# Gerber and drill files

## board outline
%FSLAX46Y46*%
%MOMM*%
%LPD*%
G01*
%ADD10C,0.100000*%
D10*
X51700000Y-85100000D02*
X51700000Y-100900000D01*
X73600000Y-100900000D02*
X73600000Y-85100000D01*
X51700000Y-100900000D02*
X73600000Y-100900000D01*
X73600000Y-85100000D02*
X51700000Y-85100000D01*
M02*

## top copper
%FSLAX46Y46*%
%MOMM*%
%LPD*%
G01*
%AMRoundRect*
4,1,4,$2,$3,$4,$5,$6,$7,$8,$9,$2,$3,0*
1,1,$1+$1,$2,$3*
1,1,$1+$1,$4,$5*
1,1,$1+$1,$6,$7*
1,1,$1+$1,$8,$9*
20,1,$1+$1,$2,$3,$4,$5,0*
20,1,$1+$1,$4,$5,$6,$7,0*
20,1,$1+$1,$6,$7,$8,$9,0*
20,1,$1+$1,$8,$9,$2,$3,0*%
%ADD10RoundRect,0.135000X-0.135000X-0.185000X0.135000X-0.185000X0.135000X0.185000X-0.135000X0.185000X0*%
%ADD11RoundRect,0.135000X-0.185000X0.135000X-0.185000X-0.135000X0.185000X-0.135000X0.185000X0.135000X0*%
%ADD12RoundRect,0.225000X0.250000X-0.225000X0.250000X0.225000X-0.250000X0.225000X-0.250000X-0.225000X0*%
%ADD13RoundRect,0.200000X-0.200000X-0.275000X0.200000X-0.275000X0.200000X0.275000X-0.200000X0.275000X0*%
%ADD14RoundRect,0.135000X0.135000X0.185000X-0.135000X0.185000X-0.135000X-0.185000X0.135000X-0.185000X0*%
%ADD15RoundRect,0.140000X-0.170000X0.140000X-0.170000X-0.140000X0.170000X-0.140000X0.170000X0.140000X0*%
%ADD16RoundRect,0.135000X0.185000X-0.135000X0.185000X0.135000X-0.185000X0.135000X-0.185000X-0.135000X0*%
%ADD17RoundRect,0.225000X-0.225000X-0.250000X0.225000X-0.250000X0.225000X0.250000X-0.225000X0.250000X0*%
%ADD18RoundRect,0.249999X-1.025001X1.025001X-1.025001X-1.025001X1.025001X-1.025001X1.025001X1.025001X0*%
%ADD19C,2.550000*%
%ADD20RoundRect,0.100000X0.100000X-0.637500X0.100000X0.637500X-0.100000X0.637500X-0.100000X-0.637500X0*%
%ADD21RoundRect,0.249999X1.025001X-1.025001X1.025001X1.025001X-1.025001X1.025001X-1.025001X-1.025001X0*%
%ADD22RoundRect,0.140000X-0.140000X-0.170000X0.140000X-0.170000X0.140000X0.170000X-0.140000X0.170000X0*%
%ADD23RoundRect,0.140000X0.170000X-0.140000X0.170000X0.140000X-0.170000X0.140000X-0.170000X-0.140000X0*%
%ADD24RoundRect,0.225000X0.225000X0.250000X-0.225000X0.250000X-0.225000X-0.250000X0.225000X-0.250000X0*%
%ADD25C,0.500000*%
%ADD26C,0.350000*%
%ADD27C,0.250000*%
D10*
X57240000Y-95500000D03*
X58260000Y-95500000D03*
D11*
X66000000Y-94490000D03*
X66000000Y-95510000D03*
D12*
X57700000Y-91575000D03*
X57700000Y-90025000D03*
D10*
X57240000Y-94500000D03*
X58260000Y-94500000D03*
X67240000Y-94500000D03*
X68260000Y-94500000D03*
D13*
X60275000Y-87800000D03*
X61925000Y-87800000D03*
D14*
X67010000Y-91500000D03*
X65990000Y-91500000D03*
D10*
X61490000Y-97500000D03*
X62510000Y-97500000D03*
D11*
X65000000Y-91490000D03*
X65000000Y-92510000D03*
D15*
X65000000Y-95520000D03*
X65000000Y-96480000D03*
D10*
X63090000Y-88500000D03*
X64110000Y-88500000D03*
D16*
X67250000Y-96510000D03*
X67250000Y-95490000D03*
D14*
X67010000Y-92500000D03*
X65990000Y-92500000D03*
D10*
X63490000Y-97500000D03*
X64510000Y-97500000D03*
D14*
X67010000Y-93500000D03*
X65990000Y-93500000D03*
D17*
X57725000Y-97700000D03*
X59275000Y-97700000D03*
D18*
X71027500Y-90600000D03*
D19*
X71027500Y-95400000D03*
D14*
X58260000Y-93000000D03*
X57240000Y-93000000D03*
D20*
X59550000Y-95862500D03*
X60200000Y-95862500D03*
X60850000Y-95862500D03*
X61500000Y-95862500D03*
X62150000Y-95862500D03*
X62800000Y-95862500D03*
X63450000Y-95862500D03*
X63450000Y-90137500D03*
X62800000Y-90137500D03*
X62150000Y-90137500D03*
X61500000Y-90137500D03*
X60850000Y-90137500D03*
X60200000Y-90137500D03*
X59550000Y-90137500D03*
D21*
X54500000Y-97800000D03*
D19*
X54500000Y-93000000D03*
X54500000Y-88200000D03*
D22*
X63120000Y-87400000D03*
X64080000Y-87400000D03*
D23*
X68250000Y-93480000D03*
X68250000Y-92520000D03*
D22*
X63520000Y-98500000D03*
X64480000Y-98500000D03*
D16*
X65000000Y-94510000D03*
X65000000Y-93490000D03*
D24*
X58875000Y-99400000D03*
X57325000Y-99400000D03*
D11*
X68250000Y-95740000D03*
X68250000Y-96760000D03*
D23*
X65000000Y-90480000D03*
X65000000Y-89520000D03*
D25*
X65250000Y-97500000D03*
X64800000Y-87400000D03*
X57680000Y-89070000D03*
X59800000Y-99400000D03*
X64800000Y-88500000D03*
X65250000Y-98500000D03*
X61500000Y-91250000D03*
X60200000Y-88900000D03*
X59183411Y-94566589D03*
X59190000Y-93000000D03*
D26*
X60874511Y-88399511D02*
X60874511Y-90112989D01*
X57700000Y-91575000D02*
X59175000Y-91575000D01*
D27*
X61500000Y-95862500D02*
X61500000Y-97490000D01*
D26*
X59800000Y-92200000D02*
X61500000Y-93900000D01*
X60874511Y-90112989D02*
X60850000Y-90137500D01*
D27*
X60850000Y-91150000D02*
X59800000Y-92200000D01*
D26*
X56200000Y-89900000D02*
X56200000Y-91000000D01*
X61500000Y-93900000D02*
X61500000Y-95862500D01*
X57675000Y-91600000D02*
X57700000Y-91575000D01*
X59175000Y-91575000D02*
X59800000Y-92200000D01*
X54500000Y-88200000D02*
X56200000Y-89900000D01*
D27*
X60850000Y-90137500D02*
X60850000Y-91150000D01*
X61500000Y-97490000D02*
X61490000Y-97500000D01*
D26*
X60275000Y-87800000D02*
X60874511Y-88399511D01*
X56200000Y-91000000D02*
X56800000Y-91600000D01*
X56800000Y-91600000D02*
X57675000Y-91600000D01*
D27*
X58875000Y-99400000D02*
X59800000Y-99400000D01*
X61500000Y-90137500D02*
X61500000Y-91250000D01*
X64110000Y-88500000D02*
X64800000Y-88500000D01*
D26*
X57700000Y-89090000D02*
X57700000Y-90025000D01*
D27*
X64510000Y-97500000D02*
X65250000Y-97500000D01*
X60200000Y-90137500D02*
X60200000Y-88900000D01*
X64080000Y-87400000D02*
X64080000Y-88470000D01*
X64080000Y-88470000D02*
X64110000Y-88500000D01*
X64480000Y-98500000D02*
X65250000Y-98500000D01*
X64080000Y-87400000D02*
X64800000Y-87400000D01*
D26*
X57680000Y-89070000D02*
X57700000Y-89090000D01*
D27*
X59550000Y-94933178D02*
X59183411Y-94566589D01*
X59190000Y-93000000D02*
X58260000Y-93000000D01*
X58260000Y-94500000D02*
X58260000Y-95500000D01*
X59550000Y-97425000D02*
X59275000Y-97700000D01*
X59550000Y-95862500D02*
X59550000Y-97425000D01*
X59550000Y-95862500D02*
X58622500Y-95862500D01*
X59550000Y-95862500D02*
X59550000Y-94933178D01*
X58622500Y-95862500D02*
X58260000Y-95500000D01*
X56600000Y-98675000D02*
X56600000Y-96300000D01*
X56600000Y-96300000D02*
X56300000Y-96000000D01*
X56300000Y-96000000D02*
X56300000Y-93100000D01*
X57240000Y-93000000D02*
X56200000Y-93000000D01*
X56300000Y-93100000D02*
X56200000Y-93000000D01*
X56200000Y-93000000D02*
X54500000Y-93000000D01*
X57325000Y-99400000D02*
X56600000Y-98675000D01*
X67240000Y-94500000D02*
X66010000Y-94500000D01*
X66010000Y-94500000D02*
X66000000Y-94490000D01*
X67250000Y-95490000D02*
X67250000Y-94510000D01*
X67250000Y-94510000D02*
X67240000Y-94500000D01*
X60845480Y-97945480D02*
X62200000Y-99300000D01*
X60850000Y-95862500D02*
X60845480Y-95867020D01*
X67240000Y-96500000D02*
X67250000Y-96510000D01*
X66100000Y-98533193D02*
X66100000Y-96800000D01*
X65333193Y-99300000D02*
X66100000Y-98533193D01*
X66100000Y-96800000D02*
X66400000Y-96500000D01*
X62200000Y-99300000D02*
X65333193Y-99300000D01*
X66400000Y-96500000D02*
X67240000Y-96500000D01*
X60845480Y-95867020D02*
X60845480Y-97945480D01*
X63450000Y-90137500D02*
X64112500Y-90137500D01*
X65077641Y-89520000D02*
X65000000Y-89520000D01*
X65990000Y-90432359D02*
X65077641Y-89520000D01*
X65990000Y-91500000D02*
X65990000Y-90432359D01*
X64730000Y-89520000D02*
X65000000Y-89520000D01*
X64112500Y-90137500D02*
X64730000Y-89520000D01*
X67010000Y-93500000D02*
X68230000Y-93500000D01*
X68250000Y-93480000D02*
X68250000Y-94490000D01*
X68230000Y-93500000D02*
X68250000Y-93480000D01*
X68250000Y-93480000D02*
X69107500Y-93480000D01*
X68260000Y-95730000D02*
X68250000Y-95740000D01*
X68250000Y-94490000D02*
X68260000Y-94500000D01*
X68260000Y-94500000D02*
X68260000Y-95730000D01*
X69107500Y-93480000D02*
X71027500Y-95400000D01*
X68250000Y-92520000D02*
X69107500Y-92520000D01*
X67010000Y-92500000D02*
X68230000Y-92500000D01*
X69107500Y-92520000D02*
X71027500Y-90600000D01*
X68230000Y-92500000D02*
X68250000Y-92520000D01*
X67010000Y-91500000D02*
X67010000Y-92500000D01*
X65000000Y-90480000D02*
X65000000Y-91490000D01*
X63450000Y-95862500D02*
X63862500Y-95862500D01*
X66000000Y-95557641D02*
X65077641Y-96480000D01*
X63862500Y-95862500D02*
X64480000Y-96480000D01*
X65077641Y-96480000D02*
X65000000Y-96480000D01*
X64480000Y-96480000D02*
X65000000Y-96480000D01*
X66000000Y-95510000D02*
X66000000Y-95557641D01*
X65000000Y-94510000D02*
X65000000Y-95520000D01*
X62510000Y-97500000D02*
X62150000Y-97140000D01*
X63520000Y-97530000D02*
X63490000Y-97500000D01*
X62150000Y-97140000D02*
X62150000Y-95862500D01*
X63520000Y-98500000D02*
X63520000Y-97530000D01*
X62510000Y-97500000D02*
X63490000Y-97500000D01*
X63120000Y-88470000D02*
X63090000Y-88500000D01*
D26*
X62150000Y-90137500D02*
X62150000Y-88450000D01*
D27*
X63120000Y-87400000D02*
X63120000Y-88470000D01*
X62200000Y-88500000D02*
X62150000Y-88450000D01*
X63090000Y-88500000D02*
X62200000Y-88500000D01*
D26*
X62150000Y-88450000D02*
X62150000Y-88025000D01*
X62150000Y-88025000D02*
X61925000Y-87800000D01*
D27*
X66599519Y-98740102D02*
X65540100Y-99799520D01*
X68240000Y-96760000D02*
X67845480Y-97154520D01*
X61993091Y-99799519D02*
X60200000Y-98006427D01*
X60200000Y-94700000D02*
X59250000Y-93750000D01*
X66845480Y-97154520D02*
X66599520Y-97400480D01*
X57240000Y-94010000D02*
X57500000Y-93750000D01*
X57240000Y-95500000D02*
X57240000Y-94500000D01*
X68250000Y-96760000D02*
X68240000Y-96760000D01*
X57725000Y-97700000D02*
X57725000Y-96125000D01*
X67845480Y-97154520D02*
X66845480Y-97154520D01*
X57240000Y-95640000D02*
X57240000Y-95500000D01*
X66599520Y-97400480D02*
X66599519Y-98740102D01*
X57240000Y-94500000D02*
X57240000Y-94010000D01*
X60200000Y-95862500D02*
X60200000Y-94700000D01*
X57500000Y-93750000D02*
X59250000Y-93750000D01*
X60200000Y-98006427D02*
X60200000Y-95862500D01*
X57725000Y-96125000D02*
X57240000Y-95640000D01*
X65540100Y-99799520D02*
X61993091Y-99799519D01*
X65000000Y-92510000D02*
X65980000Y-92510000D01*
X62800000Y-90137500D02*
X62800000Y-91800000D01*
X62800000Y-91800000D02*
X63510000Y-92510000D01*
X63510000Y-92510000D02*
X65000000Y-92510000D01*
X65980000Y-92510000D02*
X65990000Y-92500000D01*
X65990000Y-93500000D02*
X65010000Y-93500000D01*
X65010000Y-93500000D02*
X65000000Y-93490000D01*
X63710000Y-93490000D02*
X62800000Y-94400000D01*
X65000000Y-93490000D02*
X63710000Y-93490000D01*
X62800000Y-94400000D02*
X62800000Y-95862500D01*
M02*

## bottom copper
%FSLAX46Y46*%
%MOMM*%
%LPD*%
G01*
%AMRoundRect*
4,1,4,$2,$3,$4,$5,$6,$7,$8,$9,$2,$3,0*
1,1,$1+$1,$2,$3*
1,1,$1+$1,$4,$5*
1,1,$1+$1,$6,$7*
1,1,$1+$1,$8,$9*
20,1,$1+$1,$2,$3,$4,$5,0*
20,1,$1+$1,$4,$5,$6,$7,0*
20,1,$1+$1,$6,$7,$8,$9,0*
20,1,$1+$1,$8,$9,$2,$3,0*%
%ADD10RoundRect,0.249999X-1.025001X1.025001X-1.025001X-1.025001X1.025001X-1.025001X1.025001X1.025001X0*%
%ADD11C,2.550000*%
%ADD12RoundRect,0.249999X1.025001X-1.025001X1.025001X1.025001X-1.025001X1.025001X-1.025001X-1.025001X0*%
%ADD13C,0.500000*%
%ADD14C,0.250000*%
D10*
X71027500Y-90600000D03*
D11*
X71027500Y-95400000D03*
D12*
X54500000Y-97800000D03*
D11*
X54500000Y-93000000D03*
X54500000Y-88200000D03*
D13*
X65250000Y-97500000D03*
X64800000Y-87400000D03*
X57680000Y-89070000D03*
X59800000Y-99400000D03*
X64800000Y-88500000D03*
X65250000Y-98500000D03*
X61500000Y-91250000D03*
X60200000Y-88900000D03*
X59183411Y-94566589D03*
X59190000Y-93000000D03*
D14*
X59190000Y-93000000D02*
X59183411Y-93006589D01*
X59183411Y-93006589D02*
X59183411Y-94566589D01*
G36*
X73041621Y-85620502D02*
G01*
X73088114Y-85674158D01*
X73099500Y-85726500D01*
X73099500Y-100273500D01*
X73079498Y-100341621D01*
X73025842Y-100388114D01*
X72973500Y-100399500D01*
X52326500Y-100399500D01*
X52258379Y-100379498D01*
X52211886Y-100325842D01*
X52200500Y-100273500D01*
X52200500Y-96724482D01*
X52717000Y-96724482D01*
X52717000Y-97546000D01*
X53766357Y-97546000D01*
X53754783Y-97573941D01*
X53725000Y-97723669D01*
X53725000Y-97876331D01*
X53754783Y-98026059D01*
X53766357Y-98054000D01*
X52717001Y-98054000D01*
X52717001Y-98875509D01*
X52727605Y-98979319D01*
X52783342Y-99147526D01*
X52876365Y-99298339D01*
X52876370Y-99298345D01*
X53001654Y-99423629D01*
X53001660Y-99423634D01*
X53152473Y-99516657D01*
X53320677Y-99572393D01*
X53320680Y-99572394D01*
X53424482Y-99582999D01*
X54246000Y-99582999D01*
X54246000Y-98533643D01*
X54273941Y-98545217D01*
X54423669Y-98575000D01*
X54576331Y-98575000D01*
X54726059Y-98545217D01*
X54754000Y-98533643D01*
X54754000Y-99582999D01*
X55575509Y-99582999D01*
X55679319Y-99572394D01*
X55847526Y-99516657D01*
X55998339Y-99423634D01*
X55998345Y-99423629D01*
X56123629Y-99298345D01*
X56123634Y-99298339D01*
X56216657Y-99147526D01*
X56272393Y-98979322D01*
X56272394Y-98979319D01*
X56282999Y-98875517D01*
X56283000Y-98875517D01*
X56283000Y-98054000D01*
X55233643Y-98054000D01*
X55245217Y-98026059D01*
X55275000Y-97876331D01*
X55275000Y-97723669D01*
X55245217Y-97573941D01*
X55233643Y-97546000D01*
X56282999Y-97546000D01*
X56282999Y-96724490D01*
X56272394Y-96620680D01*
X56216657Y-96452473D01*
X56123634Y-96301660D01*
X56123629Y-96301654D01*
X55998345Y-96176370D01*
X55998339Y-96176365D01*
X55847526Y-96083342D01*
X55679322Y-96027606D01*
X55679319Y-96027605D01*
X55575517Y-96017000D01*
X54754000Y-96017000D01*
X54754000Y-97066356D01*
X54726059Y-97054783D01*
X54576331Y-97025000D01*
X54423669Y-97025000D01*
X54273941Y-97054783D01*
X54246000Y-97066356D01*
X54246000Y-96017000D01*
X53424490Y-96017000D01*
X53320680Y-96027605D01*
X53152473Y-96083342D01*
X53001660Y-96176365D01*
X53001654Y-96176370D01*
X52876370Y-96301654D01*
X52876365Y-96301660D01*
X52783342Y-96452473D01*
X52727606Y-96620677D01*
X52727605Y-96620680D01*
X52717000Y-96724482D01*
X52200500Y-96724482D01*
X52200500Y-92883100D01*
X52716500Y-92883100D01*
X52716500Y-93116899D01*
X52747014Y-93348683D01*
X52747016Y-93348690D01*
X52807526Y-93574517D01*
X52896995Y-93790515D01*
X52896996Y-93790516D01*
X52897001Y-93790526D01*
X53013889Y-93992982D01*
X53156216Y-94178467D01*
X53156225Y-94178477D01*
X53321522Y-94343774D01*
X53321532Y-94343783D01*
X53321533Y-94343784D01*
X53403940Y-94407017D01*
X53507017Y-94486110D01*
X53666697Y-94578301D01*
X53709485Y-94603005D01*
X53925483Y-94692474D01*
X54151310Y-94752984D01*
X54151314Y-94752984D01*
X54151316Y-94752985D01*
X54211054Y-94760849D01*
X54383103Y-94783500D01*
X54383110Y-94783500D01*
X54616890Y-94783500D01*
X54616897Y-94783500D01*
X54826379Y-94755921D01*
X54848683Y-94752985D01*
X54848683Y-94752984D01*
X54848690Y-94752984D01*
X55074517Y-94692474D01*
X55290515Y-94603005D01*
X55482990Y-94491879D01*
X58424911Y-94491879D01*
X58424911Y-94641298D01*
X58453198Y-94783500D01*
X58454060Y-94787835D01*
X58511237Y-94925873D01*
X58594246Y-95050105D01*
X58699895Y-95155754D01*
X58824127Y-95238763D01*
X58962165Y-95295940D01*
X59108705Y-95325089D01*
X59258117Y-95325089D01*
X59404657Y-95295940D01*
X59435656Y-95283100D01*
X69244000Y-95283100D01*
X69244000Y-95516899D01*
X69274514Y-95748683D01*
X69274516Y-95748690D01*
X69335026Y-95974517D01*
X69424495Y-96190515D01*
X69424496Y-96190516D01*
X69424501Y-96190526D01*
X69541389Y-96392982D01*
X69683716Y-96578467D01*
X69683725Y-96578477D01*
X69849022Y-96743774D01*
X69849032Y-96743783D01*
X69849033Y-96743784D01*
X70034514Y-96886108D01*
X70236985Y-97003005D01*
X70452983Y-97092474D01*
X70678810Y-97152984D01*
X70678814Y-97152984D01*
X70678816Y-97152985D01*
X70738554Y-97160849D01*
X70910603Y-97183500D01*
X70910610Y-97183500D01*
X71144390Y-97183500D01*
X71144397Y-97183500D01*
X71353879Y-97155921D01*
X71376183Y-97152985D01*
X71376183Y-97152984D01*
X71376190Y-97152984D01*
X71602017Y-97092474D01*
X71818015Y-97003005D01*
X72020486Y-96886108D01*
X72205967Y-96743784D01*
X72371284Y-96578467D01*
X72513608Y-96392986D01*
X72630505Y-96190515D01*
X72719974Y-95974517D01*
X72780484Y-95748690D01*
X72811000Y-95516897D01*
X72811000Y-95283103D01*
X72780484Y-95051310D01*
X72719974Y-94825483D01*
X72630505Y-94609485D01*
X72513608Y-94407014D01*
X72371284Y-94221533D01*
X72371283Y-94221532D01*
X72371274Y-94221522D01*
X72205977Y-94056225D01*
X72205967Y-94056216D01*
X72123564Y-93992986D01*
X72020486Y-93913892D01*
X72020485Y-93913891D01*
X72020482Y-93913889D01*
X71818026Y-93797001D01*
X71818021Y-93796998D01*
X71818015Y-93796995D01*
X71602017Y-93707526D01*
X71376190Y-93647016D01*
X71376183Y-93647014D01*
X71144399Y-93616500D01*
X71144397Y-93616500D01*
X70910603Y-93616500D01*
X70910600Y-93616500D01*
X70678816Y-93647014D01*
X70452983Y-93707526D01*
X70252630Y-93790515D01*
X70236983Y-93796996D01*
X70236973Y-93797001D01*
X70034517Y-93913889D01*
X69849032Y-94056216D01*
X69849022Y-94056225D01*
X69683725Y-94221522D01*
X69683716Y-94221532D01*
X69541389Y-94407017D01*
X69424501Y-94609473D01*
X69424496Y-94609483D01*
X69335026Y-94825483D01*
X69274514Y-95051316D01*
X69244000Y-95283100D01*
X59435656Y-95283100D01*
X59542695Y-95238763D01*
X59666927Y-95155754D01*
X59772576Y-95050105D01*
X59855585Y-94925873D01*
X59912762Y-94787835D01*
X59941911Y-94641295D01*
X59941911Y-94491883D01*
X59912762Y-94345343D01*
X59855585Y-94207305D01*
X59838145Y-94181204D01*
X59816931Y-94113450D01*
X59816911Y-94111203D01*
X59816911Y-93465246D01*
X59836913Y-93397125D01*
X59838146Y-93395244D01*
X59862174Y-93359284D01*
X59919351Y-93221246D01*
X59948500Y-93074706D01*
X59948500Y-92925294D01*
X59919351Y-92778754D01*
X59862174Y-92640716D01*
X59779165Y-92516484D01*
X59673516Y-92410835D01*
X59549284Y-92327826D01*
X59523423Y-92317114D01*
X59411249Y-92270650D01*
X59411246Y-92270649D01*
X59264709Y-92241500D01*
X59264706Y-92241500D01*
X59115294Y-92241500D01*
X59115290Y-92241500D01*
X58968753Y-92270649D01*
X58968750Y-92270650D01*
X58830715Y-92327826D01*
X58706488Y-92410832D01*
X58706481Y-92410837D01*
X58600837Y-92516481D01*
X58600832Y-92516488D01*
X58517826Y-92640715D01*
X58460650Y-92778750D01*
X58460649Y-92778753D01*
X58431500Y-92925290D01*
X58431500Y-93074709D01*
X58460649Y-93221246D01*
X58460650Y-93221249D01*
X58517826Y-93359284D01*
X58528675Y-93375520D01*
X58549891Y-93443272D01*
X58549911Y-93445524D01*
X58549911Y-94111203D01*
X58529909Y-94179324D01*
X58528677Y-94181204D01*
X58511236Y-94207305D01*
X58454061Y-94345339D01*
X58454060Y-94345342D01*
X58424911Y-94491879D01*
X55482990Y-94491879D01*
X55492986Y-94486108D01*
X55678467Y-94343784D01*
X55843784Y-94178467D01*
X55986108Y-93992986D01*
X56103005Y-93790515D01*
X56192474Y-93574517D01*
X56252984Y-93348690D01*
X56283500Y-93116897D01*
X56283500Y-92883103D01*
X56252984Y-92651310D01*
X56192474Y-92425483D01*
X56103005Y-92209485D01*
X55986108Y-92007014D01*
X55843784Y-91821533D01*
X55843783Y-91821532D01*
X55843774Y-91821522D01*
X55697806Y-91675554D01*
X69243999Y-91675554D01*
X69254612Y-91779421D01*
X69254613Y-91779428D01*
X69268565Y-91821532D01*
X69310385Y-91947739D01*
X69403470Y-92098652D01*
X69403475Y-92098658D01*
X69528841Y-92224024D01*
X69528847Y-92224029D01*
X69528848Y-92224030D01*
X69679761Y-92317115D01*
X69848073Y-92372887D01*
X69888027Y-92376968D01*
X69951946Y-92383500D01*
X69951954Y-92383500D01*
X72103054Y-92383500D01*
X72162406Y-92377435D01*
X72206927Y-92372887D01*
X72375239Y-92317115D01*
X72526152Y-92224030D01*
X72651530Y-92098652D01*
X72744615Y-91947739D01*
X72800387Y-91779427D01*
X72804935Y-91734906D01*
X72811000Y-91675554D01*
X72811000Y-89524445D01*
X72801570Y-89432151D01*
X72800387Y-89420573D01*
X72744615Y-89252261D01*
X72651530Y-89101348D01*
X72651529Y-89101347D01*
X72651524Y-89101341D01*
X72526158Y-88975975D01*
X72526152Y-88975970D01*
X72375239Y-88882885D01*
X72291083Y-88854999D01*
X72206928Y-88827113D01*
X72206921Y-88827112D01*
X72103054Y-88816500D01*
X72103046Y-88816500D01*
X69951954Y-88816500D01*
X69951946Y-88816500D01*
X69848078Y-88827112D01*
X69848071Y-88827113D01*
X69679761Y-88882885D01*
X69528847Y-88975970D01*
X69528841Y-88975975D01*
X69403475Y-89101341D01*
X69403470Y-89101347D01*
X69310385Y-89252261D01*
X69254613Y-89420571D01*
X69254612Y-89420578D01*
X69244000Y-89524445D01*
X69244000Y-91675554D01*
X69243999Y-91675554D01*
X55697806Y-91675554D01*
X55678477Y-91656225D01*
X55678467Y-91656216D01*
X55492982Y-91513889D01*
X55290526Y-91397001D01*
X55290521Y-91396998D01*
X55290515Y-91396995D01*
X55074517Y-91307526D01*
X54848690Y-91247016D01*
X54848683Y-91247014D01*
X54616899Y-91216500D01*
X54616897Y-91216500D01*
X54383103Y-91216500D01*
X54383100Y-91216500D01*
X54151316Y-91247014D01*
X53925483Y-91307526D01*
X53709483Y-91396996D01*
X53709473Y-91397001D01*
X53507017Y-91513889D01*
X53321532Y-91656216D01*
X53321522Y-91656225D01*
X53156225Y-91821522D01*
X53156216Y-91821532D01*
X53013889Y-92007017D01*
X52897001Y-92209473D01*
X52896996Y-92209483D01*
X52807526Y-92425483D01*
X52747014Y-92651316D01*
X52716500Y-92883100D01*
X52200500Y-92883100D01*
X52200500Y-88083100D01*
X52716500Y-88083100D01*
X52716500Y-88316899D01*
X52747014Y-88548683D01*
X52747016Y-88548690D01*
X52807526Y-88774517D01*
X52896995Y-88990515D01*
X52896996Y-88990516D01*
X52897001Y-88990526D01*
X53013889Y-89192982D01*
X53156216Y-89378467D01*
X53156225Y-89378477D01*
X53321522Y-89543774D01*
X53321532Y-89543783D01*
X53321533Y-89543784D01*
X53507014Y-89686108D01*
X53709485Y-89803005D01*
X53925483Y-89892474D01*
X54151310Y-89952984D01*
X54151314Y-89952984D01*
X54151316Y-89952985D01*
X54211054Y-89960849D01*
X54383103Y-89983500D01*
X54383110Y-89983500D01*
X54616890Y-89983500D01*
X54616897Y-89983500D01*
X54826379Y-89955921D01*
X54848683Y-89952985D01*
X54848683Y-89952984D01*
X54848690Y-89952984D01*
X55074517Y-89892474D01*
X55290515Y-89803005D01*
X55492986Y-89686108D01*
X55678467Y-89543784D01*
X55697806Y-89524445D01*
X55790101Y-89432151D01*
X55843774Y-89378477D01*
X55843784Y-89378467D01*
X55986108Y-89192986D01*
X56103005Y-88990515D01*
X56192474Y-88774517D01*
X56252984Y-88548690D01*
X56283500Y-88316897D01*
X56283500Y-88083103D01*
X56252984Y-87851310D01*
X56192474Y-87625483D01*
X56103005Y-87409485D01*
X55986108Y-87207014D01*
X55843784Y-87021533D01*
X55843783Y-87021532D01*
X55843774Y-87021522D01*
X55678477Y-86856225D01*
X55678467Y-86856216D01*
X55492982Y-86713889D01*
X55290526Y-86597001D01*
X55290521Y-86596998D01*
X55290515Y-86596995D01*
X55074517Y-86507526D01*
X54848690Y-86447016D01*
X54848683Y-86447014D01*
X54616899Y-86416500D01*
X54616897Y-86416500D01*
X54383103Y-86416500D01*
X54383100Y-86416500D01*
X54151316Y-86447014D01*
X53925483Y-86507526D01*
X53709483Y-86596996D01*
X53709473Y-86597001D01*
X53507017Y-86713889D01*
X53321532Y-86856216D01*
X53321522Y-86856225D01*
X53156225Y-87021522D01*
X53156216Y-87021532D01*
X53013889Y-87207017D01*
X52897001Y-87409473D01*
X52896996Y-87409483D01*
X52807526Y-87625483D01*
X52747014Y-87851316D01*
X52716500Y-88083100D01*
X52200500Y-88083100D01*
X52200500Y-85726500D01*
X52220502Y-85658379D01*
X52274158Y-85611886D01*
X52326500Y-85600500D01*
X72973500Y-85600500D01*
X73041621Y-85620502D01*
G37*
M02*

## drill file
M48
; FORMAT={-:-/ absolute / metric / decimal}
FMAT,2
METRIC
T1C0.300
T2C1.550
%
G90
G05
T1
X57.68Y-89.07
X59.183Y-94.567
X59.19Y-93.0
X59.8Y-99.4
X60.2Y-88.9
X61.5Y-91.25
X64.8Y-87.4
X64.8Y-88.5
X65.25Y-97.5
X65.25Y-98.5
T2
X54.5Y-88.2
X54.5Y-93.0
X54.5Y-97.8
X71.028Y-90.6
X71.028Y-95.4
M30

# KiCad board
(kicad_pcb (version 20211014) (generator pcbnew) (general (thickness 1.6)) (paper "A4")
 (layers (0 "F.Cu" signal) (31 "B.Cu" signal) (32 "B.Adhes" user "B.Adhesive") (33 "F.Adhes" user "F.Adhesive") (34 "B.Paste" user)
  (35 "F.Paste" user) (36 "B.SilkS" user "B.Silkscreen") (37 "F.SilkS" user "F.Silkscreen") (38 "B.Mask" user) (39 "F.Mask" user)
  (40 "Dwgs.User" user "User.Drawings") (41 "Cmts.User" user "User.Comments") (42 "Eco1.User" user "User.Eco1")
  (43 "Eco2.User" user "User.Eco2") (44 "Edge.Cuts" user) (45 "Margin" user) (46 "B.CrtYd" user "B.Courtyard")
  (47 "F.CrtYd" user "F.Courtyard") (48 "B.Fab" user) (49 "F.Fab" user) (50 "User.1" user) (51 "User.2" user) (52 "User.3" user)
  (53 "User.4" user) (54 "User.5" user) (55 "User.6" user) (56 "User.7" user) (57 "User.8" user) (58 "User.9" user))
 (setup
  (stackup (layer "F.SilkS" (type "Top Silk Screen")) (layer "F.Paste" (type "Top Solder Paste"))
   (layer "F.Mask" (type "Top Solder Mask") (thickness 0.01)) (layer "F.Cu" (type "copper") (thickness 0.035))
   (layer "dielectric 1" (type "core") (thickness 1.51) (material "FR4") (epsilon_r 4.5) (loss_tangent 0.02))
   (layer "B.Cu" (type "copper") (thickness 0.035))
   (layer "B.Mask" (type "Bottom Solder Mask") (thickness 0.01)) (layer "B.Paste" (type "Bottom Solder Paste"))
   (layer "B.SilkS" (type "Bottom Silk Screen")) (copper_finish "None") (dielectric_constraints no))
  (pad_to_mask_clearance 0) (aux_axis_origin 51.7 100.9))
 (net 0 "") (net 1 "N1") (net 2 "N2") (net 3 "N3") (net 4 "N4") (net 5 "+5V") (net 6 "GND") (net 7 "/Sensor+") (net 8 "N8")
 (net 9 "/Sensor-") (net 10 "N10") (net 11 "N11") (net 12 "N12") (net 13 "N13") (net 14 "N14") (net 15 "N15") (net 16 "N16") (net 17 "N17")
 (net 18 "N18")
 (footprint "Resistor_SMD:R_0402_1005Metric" (layer "F.Cu") (at 57.75 95.5)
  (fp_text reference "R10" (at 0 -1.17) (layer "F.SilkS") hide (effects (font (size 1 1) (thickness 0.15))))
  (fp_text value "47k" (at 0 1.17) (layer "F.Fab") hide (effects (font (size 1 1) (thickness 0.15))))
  (pad "1" smd roundrect locked (at -0.51 0) (size 0.54 0.64) (layers "F.Cu" "F.Paste" "F.Mask") (roundrect_rratio 0.25) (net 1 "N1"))
  (pad "2" smd roundrect locked (at 0.51 0) (size 0.54 0.64) (layers "F.Cu" "F.Paste" "F.Mask") (roundrect_rratio 0.25) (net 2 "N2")))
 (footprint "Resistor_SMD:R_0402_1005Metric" (layer "F.Cu") (at 66 95 -90)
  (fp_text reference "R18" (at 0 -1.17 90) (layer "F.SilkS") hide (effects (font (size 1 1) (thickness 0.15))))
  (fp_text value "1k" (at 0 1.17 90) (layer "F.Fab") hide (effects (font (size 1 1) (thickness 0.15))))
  (pad "1" smd roundrect locked (at -0.51 0 270) (size 0.54 0.64) (layers "F.Cu" "F.Paste" "F.Mask") (roundrect_rratio 0.25) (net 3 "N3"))
  (pad "2" smd roundrect locked (at 0.51 0 270) (size 0.54 0.64) (layers "F.Cu" "F.Paste" "F.Mask") (roundrect_rratio 0.25) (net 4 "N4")))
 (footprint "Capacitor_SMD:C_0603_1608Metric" (layer "F.Cu") (at 57.7 90.8 90)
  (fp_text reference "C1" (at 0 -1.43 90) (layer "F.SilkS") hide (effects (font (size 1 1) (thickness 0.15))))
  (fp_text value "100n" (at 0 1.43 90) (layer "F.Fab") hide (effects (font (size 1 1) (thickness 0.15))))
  (pad "1" smd roundrect locked (at -0.775 0 90) (size 0.9 0.95) (layers "F.Cu" "F.Paste" "F.Mask") (roundrect_rratio 0.25) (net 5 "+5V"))
  (pad "2" smd roundrect locked (at 0.775 0 90) (size 0.9 0.95) (layers "F.Cu" "F.Paste" "F.Mask") (roundrect_rratio 0.25) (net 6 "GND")))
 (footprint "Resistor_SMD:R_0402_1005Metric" (layer "F.Cu") (at 57.75 94.5)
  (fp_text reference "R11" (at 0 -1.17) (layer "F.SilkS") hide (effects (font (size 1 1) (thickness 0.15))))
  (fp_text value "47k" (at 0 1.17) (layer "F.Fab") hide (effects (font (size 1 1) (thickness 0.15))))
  (pad "1" smd roundrect locked (at -0.51 0) (size 0.54 0.64) (layers "F.Cu" "F.Paste" "F.Mask") (roundrect_rratio 0.25) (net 1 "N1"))
  (pad "2" smd roundrect locked (at 0.51 0) (size 0.54 0.64) (layers "F.Cu" "F.Paste" "F.Mask") (roundrect_rratio 0.25) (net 2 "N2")))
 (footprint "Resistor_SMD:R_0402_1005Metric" (layer "F.Cu") (at 67.75 94.5)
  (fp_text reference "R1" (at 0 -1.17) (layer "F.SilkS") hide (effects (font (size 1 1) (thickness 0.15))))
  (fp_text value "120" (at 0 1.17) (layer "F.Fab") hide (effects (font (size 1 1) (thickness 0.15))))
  (pad "1" smd roundrect locked (at -0.51 0) (size 0.54 0.64) (layers "F.Cu" "F.Paste" "F.Mask") (roundrect_rratio 0.25) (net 3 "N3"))
  (pad "2" smd roundrect locked (at 0.51 0) (size 0.54 0.64) (layers "F.Cu" "F.Paste" "F.Mask") (roundrect_rratio 0.25) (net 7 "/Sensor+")))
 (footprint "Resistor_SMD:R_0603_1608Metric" (layer "F.Cu") (at 61.1 87.8)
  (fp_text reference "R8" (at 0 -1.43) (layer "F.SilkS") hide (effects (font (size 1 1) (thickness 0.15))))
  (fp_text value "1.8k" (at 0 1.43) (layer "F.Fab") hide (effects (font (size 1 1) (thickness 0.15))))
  (pad "1" smd roundrect locked (at -0.825 0) (size 0.8 0.95) (layers "F.Cu" "F.Paste" "F.Mask") (roundrect_rratio 0.25) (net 5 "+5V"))
  (pad "2" smd roundrect locked (at 0.825 0) (size 0.8 0.95) (layers "F.Cu" "F.Paste" "F.Mask") (roundrect_rratio 0.25) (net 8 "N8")))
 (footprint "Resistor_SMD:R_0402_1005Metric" (layer "F.Cu") (at 66.5 91.5 180)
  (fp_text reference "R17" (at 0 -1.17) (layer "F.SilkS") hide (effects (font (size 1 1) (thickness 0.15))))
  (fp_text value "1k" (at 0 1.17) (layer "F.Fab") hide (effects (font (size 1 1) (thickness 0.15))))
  (pad "1" smd roundrect locked (at -0.51 0 180) (size 0.54 0.64) (layers "F.Cu" "F.Paste" "F.Mask") (roundrect_rratio 0.25)
   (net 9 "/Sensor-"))
  (pad "2" smd roundrect locked (at 0.51 0 180) (size 0.54 0.64) (layers "F.Cu" "F.Paste" "F.Mask") (roundrect_rratio 0.25) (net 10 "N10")))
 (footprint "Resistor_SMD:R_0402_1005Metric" (layer "F.Cu") (at 62 97.5)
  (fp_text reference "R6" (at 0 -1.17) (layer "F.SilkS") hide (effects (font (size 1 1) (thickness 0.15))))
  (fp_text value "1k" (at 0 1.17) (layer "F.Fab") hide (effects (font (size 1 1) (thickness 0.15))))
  (pad "1" smd roundrect locked (at -0.51 0) (size 0.54 0.64) (layers "F.Cu" "F.Paste" "F.Mask") (roundrect_rratio 0.25) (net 5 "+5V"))
  (pad "2" smd roundrect locked (at 0.51 0) (size 0.54 0.64) (layers "F.Cu" "F.Paste" "F.Mask") (roundrect_rratio 0.25) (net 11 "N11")))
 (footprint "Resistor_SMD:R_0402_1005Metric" (layer "F.Cu") (at 65 92 -90)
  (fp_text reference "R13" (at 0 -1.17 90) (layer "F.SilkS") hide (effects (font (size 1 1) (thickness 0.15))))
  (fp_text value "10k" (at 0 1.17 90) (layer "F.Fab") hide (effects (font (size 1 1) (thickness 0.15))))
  (pad "1" smd roundrect locked (at -0.51 0 270) (size 0.54 0.64) (layers "F.Cu" "F.Paste" "F.Mask") (roundrect_rratio 0.25) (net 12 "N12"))
  (pad "2" smd roundrect locked (at 0.51 0 270) (size 0.54 0.64) (layers "F.Cu" "F.Paste" "F.Mask") (roundrect_rratio 0.25) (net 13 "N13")))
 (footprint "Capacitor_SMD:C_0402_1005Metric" (layer "F.Cu") (at 65 96 -90)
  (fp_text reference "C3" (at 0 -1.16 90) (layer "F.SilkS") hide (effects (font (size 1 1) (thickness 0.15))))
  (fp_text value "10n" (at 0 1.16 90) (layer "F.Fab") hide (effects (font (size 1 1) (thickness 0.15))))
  (pad "1" smd roundrect locked (at -0.48 0 270) (size 0.56 0.62) (layers "F.Cu" "F.Paste" "F.Mask") (roundrect_rratio 0.25) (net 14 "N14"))
  (pad "2" smd roundrect locked (at 0.48 0 270) (size 0.56 0.62) (layers "F.Cu" "F.Paste" "F.Mask") (roundrect_rratio 0.25) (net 4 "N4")))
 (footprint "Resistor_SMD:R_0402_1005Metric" (layer "F.Cu") (at 63.6 88.5)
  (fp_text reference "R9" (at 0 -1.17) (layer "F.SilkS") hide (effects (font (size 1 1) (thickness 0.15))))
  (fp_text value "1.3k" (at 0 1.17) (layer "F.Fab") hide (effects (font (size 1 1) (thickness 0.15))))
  (pad "1" smd roundrect locked (at -0.51 0) (size 0.54 0.64) (layers "F.Cu" "F.Paste" "F.Mask") (roundrect_rratio 0.25) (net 8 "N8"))
  (pad "2" smd roundrect locked (at 0.51 0) (size 0.54 0.64) (layers "F.Cu" "F.Paste" "F.Mask") (roundrect_rratio 0.25) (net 6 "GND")))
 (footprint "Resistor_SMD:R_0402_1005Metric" (layer "F.Cu") (at 67.25 96 90)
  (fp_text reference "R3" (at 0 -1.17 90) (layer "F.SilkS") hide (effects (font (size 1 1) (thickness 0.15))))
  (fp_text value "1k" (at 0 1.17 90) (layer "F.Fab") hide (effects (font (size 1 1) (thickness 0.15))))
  (pad "1" smd roundrect locked (at -0.51 0 90) (size 0.54 0.64) (layers "F.Cu" "F.Paste" "F.Mask") (roundrect_rratio 0.25) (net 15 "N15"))
  (pad "2" smd roundrect locked (at 0.51 0 90) (size 0.54 0.64) (layers "F.Cu" "F.Paste" "F.Mask") (roundrect_rratio 0.25) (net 3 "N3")))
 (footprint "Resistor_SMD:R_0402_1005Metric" (layer "F.Cu") (at 66.5 92.5 180)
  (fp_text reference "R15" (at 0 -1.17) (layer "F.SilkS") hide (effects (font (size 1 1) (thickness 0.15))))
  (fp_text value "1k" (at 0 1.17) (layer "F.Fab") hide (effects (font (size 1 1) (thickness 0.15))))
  (pad "1" smd roundrect locked (at -0.51 0 180) (size 0.54 0.64) (layers "F.Cu" "F.Paste" "F.Mask") (roundrect_rratio 0.25)
   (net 9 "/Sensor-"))
  (pad "2" smd roundrect locked (at 0.51 0 180) (size 0.54 0.64) (layers "F.Cu" "F.Paste" "F.Mask") (roundrect_rratio 0.25) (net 13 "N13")))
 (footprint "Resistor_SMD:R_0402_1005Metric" (layer "F.Cu") (at 64 97.5)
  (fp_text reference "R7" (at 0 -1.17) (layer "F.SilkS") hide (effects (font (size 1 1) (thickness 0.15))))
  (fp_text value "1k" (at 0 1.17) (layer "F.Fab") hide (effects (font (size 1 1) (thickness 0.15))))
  (pad "1" smd roundrect locked (at -0.51 0) (size 0.54 0.64) (layers "F.Cu" "F.Paste" "F.Mask") (roundrect_rratio 0.25) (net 11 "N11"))
  (pad "2" smd roundrect locked (at 0.51 0) (size 0.54 0.64) (layers "F.Cu" "F.Paste" "F.Mask") (roundrect_rratio 0.25) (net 6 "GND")))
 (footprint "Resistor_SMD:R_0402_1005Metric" (layer "F.Cu") (at 66.5 93.5 180)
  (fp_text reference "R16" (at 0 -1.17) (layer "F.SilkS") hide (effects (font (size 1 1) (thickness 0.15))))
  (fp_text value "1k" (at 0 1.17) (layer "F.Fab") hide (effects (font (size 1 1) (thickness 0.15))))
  (pad "1" smd roundrect locked (at -0.51 0 180) (size 0.54 0.64) (layers "F.Cu" "F.Paste" "F.Mask") (roundrect_rratio 0.25)
   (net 7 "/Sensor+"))
  (pad "2" smd roundrect locked (at 0.51 0 180) (size 0.54 0.64) (layers "F.Cu" "F.Paste" "F.Mask") (roundrect_rratio 0.25) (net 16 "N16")))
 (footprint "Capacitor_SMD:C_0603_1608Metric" (layer "F.Cu") (at 58.5 97.7)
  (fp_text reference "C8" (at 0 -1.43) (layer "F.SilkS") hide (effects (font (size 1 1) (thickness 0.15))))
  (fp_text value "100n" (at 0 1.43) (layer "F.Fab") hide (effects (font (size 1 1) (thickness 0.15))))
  (pad "1" smd roundrect locked (at -0.775 0) (size 0.9 0.95) (layers "F.Cu" "F.Paste" "F.Mask") (roundrect_rratio 0.25) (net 1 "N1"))
  (pad "2" smd roundrect locked (at 0.775 0) (size 0.9 0.95) (layers "F.Cu" "F.Paste" "F.Mask") (roundrect_rratio 0.25) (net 2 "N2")))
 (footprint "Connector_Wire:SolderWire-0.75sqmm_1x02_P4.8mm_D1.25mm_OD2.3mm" (layer "F.Cu") (at 71.0275 90.6 -90)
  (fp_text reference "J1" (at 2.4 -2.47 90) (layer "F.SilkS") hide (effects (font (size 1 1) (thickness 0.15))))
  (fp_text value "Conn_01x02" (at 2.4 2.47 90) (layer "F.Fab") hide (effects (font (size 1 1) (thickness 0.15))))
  (pad "1" thru_hole roundrect locked (at 0 0 270) (size 2.55 2.55) (drill 1.55) (layers *.Cu *.Mask) (roundrect_rratio 0.09803882353)
   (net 9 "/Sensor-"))
  (pad "2" thru_hole circle locked (at 4.8 0 270) (size 2.55 2.55) (drill 1.55) (layers *.Cu *.Mask) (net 7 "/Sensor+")))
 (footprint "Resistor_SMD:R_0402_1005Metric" (layer "F.Cu") (at 57.75 93 180)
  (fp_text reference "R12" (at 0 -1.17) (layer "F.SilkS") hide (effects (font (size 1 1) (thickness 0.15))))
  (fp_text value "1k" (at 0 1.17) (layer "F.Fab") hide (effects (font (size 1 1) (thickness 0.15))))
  (pad "1" smd roundrect locked (at -0.51 0 180) (size 0.54 0.64) (layers "F.Cu" "F.Paste" "F.Mask") (roundrect_rratio 0.25) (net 2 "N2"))
  (pad "2" smd roundrect locked (at 0.51 0 180) (size 0.54 0.64) (layers "F.Cu" "F.Paste" "F.Mask") (roundrect_rratio 0.25) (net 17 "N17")))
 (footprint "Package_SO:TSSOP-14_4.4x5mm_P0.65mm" (layer "F.Cu") (at 61.5 93 90)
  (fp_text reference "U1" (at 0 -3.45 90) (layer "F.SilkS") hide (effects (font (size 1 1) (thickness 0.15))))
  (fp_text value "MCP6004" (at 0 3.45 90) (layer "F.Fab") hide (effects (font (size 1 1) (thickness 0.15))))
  (pad "1" smd roundrect locked (at -2.8625 -1.95 90) (size 1.475 0.4) (layers "F.Cu" "F.Paste" "F.Mask") (roundrect_rratio 0.25)
   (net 2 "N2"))
  (pad "2" smd roundrect locked (at -2.8625 -1.3 90) (size 1.475 0.4) (layers "F.Cu" "F.Paste" "F.Mask") (roundrect_rratio 0.25)
   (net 1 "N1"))
  (pad "3" smd roundrect locked (at -2.8625 -0.65 90) (size 1.475 0.4) (layers "F.Cu" "F.Paste" "F.Mask") (roundrect_rratio 0.25)
   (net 15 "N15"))
  (pad "4" smd roundrect locked (at -2.8625 0 90) (size 1.475 0.4) (layers "F.Cu" "F.Paste" "F.Mask") (roundrect_rratio 0.25) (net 5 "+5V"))
  (pad "5" smd roundrect locked (at -2.8625 0.65 90) (size 1.475 0.4) (layers "F.Cu" "F.Paste" "F.Mask") (roundrect_rratio 0.25)
   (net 11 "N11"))
  (pad "6" smd roundrect locked (at -2.8625 1.3 90) (size 1.475 0.4) (layers "F.Cu" "F.Paste" "F.Mask") (roundrect_rratio 0.25)
   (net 16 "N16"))
  (pad "7" smd roundrect locked (at -2.8625 1.95 90) (size 1.475 0.4) (layers "F.Cu" "F.Paste" "F.Mask") (roundrect_rratio 0.25)
   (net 4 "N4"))
  (pad "8" smd roundrect locked (at 2.8625 1.95 90) (size 1.475 0.4) (layers "F.Cu" "F.Paste" "F.Mask") (roundrect_rratio 0.25)
   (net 10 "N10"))
  (pad "9" smd roundrect locked (at 2.8625 1.3 90) (size 1.475 0.4) (layers "F.Cu" "F.Paste" "F.Mask") (roundrect_rratio 0.25)
   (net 13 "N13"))
  (pad "10" smd roundrect locked (at 2.8625 0.65 90) (size 1.475 0.4) (layers "F.Cu" "F.Paste" "F.Mask") (roundrect_rratio 0.25)
   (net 8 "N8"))
  (pad "11" smd roundrect locked (at 2.8625 0 90) (size 1.475 0.4) (layers "F.Cu" "F.Paste" "F.Mask") (roundrect_rratio 0.25) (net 6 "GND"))
  (pad "12" smd roundrect locked (at 2.8625 -0.65 90) (size 1.475 0.4) (layers "F.Cu" "F.Paste" "F.Mask") (roundrect_rratio 0.25)
   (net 5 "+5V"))
  (pad "13" smd roundrect locked (at 2.8625 -1.3 90) (size 1.475 0.4) (layers "F.Cu" "F.Paste" "F.Mask") (roundrect_rratio 0.25)
   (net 6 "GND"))
  (pad "14" smd roundrect locked (at 2.8625 -1.95 90) (size 1.475 0.4) (layers "F.Cu" "F.Paste" "F.Mask") (roundrect_rratio 0.25)
   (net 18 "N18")))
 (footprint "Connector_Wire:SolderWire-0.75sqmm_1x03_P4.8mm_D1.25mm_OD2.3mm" (layer "F.Cu") (at 54.5 97.8 90)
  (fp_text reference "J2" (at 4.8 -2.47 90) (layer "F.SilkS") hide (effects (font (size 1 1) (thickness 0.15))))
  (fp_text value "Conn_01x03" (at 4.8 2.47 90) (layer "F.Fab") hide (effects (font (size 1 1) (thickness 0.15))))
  (pad "1" thru_hole roundrect locked (at 0 0 90) (size 2.55 2.55) (drill 1.55) (layers *.Cu *.Mask) (roundrect_rratio 0.09803882353)
   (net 6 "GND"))
  (pad "2" thru_hole circle locked (at 4.8 0 90) (size 2.55 2.55) (drill 1.55) (layers *.Cu *.Mask) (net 17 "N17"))
  (pad "3" thru_hole circle locked (at 9.6 0 90) (size 2.55 2.55) (drill 1.55) (layers *.Cu *.Mask) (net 5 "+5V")))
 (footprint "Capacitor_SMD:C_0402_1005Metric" (layer "F.Cu") (at 63.6 87.4)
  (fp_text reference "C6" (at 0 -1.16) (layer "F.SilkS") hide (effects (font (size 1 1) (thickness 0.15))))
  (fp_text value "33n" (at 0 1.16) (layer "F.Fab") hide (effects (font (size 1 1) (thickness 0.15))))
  (pad "1" smd roundrect locked (at -0.48 0) (size 0.56 0.62) (layers "F.Cu" "F.Paste" "F.Mask") (roundrect_rratio 0.25) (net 8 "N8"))
  (pad "2" smd roundrect locked (at 0.48 0) (size 0.56 0.62) (layers "F.Cu" "F.Paste" "F.Mask") (roundrect_rratio 0.25) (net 6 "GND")))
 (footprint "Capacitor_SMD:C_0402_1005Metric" (layer "F.Cu") (at 68.25 93 90)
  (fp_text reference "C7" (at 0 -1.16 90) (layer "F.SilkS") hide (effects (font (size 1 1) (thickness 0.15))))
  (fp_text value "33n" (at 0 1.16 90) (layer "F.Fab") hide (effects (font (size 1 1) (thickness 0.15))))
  (pad "1" smd roundrect locked (at -0.48 0 90) (size 0.56 0.62) (layers "F.Cu" "F.Paste" "F.Mask") (roundrect_rratio 0.25)
   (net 7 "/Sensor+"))
  (pad "2" smd roundrect locked (at 0.48 0 90) (size 0.56 0.62) (layers "F.Cu" "F.Paste" "F.Mask") (roundrect_rratio 0.25)
   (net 9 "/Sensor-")))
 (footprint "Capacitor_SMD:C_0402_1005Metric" (layer "F.Cu") (at 64 98.5)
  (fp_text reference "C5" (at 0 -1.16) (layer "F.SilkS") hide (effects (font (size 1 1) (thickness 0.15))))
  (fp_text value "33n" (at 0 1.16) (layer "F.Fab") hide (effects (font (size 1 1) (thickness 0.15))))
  (pad "1" smd roundrect locked (at -0.48 0) (size 0.56 0.62) (layers "F.Cu" "F.Paste" "F.Mask") (roundrect_rratio 0.25) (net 11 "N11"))
  (pad "2" smd roundrect locked (at 0.48 0) (size 0.56 0.62) (layers "F.Cu" "F.Paste" "F.Mask") (roundrect_rratio 0.25) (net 6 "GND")))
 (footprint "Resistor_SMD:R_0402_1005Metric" (layer "F.Cu") (at 65 94 90)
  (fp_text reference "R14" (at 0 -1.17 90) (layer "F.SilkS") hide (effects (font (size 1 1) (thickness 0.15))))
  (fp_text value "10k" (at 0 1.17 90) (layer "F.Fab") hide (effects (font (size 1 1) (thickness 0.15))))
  (pad "1" smd roundrect locked (at -0.51 0 90) (size 0.54 0.64) (layers "F.Cu" "F.Paste" "F.Mask") (roundrect_rratio 0.25) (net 14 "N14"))
  (pad "2" smd roundrect locked (at 0.51 0 90) (size 0.54 0.64) (layers "F.Cu" "F.Paste" "F.Mask") (roundrect_rratio 0.25) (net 16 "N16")))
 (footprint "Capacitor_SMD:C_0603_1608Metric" (layer "F.Cu") (at 58.1 99.4 180)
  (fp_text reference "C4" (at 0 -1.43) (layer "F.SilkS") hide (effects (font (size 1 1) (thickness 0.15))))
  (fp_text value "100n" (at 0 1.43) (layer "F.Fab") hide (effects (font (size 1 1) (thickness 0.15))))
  (pad "1" smd roundrect locked (at -0.775 0 180) (size 0.9 0.95) (layers "F.Cu" "F.Paste" "F.Mask") (roundrect_rratio 0.25) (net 6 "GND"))
  (pad "2" smd roundrect locked (at 0.775 0 180) (size 0.9 0.95) (layers "F.Cu" "F.Paste" "F.Mask") (roundrect_rratio 0.25) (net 17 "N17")))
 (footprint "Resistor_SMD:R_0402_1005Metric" (layer "F.Cu") (at 68.25 96.25 -90)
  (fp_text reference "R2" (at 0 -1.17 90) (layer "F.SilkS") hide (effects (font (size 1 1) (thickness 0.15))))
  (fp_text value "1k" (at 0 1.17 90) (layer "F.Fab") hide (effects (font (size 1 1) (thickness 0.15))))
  (pad "1" smd roundrect locked (at -0.51 0 270) (size 0.54 0.64) (layers "F.Cu" "F.Paste" "F.Mask") (roundrect_rratio 0.25)
   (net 7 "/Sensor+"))
  (pad "2" smd roundrect locked (at 0.51 0 270) (size 0.54 0.64) (layers "F.Cu" "F.Paste" "F.Mask") (roundrect_rratio 0.25) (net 1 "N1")))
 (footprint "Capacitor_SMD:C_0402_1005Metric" (layer "F.Cu") (at 65 90 90)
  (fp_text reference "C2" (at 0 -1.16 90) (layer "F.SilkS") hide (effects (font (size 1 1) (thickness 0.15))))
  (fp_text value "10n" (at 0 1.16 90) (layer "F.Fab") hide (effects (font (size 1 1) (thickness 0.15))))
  (pad "1" smd roundrect locked (at -0.48 0 90) (size 0.56 0.62) (layers "F.Cu" "F.Paste" "F.Mask") (roundrect_rratio 0.25) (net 12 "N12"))
  (pad "2" smd roundrect locked (at 0.48 0 90) (size 0.56 0.62) (layers "F.Cu" "F.Paste" "F.Mask") (roundrect_rratio 0.25) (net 10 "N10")))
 (gr_line (start 51.7 85.1) (end 51.7 100.9) (layer "Edge.Cuts") (width 0.1))
 (gr_line (start 73.6 100.9) (end 73.6 85.1) (layer "Edge.Cuts") (width 0.1))
 (gr_line (start 51.7 100.9) (end 73.6 100.9) (layer "Edge.Cuts") (width 0.1))
 (gr_line (start 73.6 85.1) (end 51.7 85.1) (layer "Edge.Cuts") (width 0.1))
 (segment (start 60.874511 88.399511) (end 60.874511 90.112989) (width 0.35) (layer "F.Cu") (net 5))
 (segment (start 57.7 91.575) (end 59.175 91.575) (width 0.35) (layer "F.Cu") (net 5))
 (segment (start 61.5 95.8625) (end 61.5 97.49) (width 0.25) (layer "F.Cu") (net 5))
 (segment (start 59.8 92.2) (end 61.5 93.9) (width 0.35) (layer "F.Cu") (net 5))
 (segment (start 60.874511 90.112989) (end 60.85 90.1375) (width 0.35) (layer "F.Cu") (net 5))
 (segment (start 60.85 91.15) (end 59.8 92.2) (width 0.25) (layer "F.Cu") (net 5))
 (segment (start 56.2 89.9) (end 56.2 91) (width 0.35) (layer "F.Cu") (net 5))
 (segment (start 61.5 93.9) (end 61.5 95.8625) (width 0.35) (layer "F.Cu") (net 5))
 (segment (start 57.675 91.6) (end 57.7 91.575) (width 0.35) (layer "F.Cu") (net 5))
 (segment (start 59.175 91.575) (end 59.8 92.2) (width 0.35) (layer "F.Cu") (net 5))
 (segment (start 54.5 88.2) (end 56.2 89.9) (width 0.35) (layer "F.Cu") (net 5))
 (segment (start 60.85 90.1375) (end 60.85 91.15) (width 0.25) (layer "F.Cu") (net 5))
 (segment (start 61.5 97.49) (end 61.49 97.5) (width 0.25) (layer "F.Cu") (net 5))
 (segment (start 60.275 87.8) (end 60.874511 88.399511) (width 0.35) (layer "F.Cu") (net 5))
 (segment (start 56.2 91) (end 56.8 91.6) (width 0.35) (layer "F.Cu") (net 5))
 (segment (start 56.8 91.6) (end 57.675 91.6) (width 0.35) (layer "F.Cu") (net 5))
 (segment (start 58.875 99.4) (end 59.8 99.4) (width 0.25) (layer "F.Cu") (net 6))
 (segment (start 61.5 90.1375) (end 61.5 91.25) (width 0.25) (layer "F.Cu") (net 6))
 (segment (start 64.11 88.5) (end 64.8 88.5) (width 0.25) (layer "F.Cu") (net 6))
 (segment (start 57.7 89.09) (end 57.7 90.025) (width 0.35) (layer "F.Cu") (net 6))
 (segment (start 64.51 97.5) (end 65.25 97.5) (width 0.25) (layer "F.Cu") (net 6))
 (segment (start 60.2 90.1375) (end 60.2 88.9) (width 0.25) (layer "F.Cu") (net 6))
 (segment (start 64.08 87.4) (end 64.08 88.47) (width 0.25) (layer "F.Cu") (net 6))
 (segment (start 64.08 88.47) (end 64.11 88.5) (width 0.25) (layer "F.Cu") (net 6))
 (segment (start 64.48 98.5) (end 65.25 98.5) (width 0.25) (layer "F.Cu") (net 6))
 (segment (start 64.08 87.4) (end 64.8 87.4) (width 0.25) (layer "F.Cu") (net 6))
 (segment (start 57.68 89.07) (end 57.7 89.09) (width 0.35) (layer "F.Cu") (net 6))
 (via (at 65.25 97.5) (size 0.5) (drill 0.3) (layers "F.Cu" "B.Cu") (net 6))
 (via (at 64.8 87.4) (size 0.5) (drill 0.3) (layers "F.Cu" "B.Cu") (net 6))
 (via (at 57.68 89.07) (size 0.5) (drill 0.3) (layers "F.Cu" "B.Cu") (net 6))
 (via (at 59.8 99.4) (size 0.5) (drill 0.3) (layers "F.Cu" "B.Cu") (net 6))
 (via (at 64.8 88.5) (size 0.5) (drill 0.3) (layers "F.Cu" "B.Cu") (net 6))
 (via (at 65.25 98.5) (size 0.5) (drill 0.3) (layers "F.Cu" "B.Cu") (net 6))
 (via (at 61.5 91.25) (size 0.5) (drill 0.3) (layers "F.Cu" "B.Cu") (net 6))
 (via (at 60.2 88.9) (size 0.5) (drill 0.3) (layers "F.Cu" "B.Cu") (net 6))
 (segment (start 59.55 94.933178) (end 59.183411 94.566589) (width 0.25) (layer "F.Cu") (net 2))
 (segment (start 59.19 93) (end 58.26 93) (width 0.25) (layer "F.Cu") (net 2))
 (segment (start 58.26 94.5) (end 58.26 95.5) (width 0.25) (layer "F.Cu") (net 2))
 (segment (start 59.55 97.425) (end 59.275 97.7) (width 0.25) (layer "F.Cu") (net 2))
 (segment (start 59.55 95.8625) (end 59.55 97.425) (width 0.25) (layer "F.Cu") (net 2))
 (segment (start 59.55 95.8625) (end 58.6225 95.8625) (width 0.25) (layer "F.Cu") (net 2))
 (segment (start 59.55 95.8625) (end 59.55 94.933178) (width 0.25) (layer "F.Cu") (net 2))
 (segment (start 58.6225 95.8625) (end 58.26 95.5) (width 0.25) (layer "F.Cu") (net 2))
 (via (at 59.183411 94.566589) (size 0.5) (drill 0.3) (layers "F.Cu" "B.Cu") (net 2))
 (via (at 59.19 93) (size 0.5) (drill 0.3) (layers "F.Cu" "B.Cu") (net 2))
 (segment (start 59.19 93) (end 59.183411 93.006589) (width 0.25) (layer "B.Cu") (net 2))
 (segment (start 59.183411 93.006589) (end 59.183411 94.566589) (width 0.25) (layer "B.Cu") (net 2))
 (segment (start 56.6 98.675) (end 56.6 96.3) (width 0.25) (layer "F.Cu") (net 17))
 (segment (start 56.6 96.3) (end 56.3 96) (width 0.25) (layer "F.Cu") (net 17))
 (segment (start 56.3 96) (end 56.3 93.1) (width 0.25) (layer "F.Cu") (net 17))
 (segment (start 57.24 93) (end 56.2 93) (width 0.25) (layer "F.Cu") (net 17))
 (segment (start 56.3 93.1) (end 56.2 93) (width 0.25) (layer "F.Cu") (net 17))
 (segment (start 56.2 93) (end 54.5 93) (width 0.25) (layer "F.Cu") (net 17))
 (segment (start 57.325 99.4) (end 56.6 98.675) (width 0.25) (layer "F.Cu") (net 17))
 (segment (start 67.24 94.5) (end 66.01 94.5) (width 0.25) (layer "F.Cu") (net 3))
 (segment (start 66.01 94.5) (end 66 94.49) (width 0.25) (layer "F.Cu") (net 3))
 (segment (start 67.25 95.49) (end 67.25 94.51) (width 0.25) (layer "F.Cu") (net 3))
 (segment (start 67.25 94.51) (end 67.24 94.5) (width 0.25) (layer "F.Cu") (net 3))
 (segment (start 60.84548 97.94548) (end 62.2 99.3) (width 0.25) (layer "F.Cu") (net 15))
 (segment (start 60.85 95.8625) (end 60.84548 95.86702) (width 0.25) (layer "F.Cu") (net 15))
 (segment (start 67.24 96.5) (end 67.25 96.51) (width 0.25) (layer "F.Cu") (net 15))
 (segment (start 66.1 98.533193) (end 66.1 96.8) (width 0.25) (layer "F.Cu") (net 15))
 (segment (start 65.333193 99.3) (end 66.1 98.533193) (width 0.25) (layer "F.Cu") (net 15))
 (segment (start 66.1 96.8) (end 66.4 96.5) (width 0.25) (layer "F.Cu") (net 15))
 (segment (start 62.2 99.3) (end 65.333193 99.3) (width 0.25) (layer "F.Cu") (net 15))
 (segment (start 66.4 96.5) (end 67.24 96.5) (width 0.25) (layer "F.Cu") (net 15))
 (segment (start 60.84548 95.86702) (end 60.84548 97.94548) (width 0.25) (layer "F.Cu") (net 15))
 (segment (start 63.45 90.1375) (end 64.1125 90.1375) (width 0.25) (layer "F.Cu") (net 10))
 (segment (start 65.077641 89.52) (end 65 89.52) (width 0.25) (layer "F.Cu") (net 10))
 (segment (start 65.99 90.432359) (end 65.077641 89.52) (width 0.25) (layer "F.Cu") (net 10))
 (segment (start 65.99 91.5) (end 65.99 90.432359) (width 0.25) (layer "F.Cu") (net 10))
 (segment (start 64.73 89.52) (end 65 89.52) (width 0.25) (layer "F.Cu") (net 10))
 (segment (start 64.1125 90.1375) (end 64.73 89.52) (width 0.25) (layer "F.Cu") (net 10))
 (segment (start 67.01 93.5) (end 68.23 93.5) (width 0.25) (layer "F.Cu") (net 7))
 (segment (start 68.25 93.48) (end 68.25 94.49) (width 0.25) (layer "F.Cu") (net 7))
 (segment (start 68.23 93.5) (end 68.25 93.48) (width 0.25) (layer "F.Cu") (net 7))
 (segment (start 68.25 93.48) (end 69.1075 93.48) (width 0.25) (layer "F.Cu") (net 7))
 (segment (start 68.26 95.73) (end 68.25 95.74) (width 0.25) (layer "F.Cu") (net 7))
 (segment (start 68.25 94.49) (end 68.26 94.5) (width 0.25) (layer "F.Cu") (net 7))
 (segment (start 68.26 94.5) (end 68.26 95.73) (width 0.25) (layer "F.Cu") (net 7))
 (segment (start 69.1075 93.48) (end 71.0275 95.4) (width 0.25) (layer "F.Cu") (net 7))
 (segment (start 68.25 92.52) (end 69.1075 92.52) (width 0.25) (layer "F.Cu") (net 9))
 (segment (start 67.01 92.5) (end 68.23 92.5) (width 0.25) (layer "F.Cu") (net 9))
 (segment (start 69.1075 92.52) (end 71.0275 90.6) (width 0.25) (layer "F.Cu") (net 9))
 (segment (start 68.23 92.5) (end 68.25 92.52) (width 0.25) (layer "F.Cu") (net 9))
 (segment (start 67.01 91.5) (end 67.01 92.5) (width 0.25) (layer "F.Cu") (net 9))
 (segment (start 65 90.48) (end 65 91.49) (width 0.25) (layer "F.Cu") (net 12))
 (segment (start 63.45 95.8625) (end 63.8625 95.8625) (width 0.25) (layer "F.Cu") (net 4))
 (segment (start 66 95.557641) (end 65.077641 96.48) (width 0.25) (layer "F.Cu") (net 4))
 (segment (start 63.8625 95.8625) (end 64.48 96.48) (width 0.25) (layer "F.Cu") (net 4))
 (segment (start 65.077641 96.48) (end 65 96.48) (width 0.25) (layer "F.Cu") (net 4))
 (segment (start 64.48 96.48) (end 65 96.48) (width 0.25) (layer "F.Cu") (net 4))
 (segment (start 66 95.51) (end 66 95.557641) (width 0.25) (layer "F.Cu") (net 4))
 (segment (start 65 94.51) (end 65 95.52) (width 0.25) (layer "F.Cu") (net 14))
 (segment (start 62.51 97.5) (end 62.15 97.14) (width 0.25) (layer "F.Cu") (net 11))
 (segment (start 63.52 97.53) (end 63.49 97.5) (width 0.25) (layer "F.Cu") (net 11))
 (segment (start 62.15 97.14) (end 62.15 95.8625) (width 0.25) (layer "F.Cu") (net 11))
 (segment (start 63.52 98.5) (end 63.52 97.53) (width 0.25) (layer "F.Cu") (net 11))
 (segment (start 62.51 97.5) (end 63.49 97.5) (width 0.25) (layer "F.Cu") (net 11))
 (segment (start 63.12 88.47) (end 63.09 88.5) (width 0.25) (layer "F.Cu") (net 8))
 (segment (start 62.15 90.1375) (end 62.15 88.45) (width 0.35) (layer "F.Cu") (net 8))
 (segment (start 63.12 87.4) (end 63.12 88.47) (width 0.25) (layer "F.Cu") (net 8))
 (segment (start 62.2 88.5) (end 62.15 88.45) (width 0.25) (layer "F.Cu") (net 8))
 (segment (start 63.09 88.5) (end 62.2 88.5) (width 0.25) (layer "F.Cu") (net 8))
 (segment (start 62.15 88.45) (end 62.15 88.025) (width 0.35) (layer "F.Cu") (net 8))
 (segment (start 62.15 88.025) (end 61.925 87.8) (width 0.35) (layer "F.Cu") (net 8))
 (segment (start 66.599519 98.740102) (end 65.5401 99.79952) (width 0.25) (layer "F.Cu") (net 1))
 (segment (start 68.24 96.76) (end 67.84548 97.15452) (width 0.25) (layer "F.Cu") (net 1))
 (segment (start 61.993091 99.799519) (end 60.2 98.006427) (width 0.25) (layer "F.Cu") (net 1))
 (segment (start 60.2 94.7) (end 59.25 93.75) (width 0.25) (layer "F.Cu") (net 1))
 (segment (start 66.84548 97.15452) (end 66.59952 97.40048) (width 0.25) (layer "F.Cu") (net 1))
 (segment (start 57.24 94.01) (end 57.5 93.75) (width 0.25) (layer "F.Cu") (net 1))
 (segment (start 57.24 95.5) (end 57.24 94.5) (width 0.25) (layer "F.Cu") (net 1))
 (segment (start 68.25 96.76) (end 68.24 96.76) (width 0.25) (layer "F.Cu") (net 1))
 (segment (start 57.725 97.7) (end 57.725 96.125) (width 0.25) (layer "F.Cu") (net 1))
 (segment (start 67.84548 97.15452) (end 66.84548 97.15452) (width 0.25) (layer "F.Cu") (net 1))
 (segment (start 57.24 95.64) (end 57.24 95.5) (width 0.25) (layer "F.Cu") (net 1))
 (segment (start 66.59952 97.40048) (end 66.599519 98.740102) (width 0.25) (layer "F.Cu") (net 1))
 (segment (start 57.24 94.5) (end 57.24 94.01) (width 0.25) (layer "F.Cu") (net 1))
 (segment (start 60.2 95.8625) (end 60.2 94.7) (width 0.25) (layer "F.Cu") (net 1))
 (segment (start 57.5 93.75) (end 59.25 93.75) (width 0.25) (layer "F.Cu") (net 1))
 (segment (start 60.2 98.006427) (end 60.2 95.8625) (width 0.25) (layer "F.Cu") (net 1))
 (segment (start 57.725 96.125) (end 57.24 95.64) (width 0.25) (layer "F.Cu") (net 1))
 (segment (start 65.5401 99.79952) (end 61.993091 99.799519) (width 0.25) (layer "F.Cu") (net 1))
 (segment (start 65 92.51) (end 65.98 92.51) (width 0.25) (layer "F.Cu") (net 13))
 (segment (start 62.8 90.1375) (end 62.8 91.8) (width 0.25) (layer "F.Cu") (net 13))
 (segment (start 62.8 91.8) (end 63.51 92.51) (width 0.25) (layer "F.Cu") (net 13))
 (segment (start 63.51 92.51) (end 65 92.51) (width 0.25) (layer "F.Cu") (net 13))
 (segment (start 65.98 92.51) (end 65.99 92.5) (width 0.25) (layer "F.Cu") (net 13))
 (segment (start 65.99 93.5) (end 65.01 93.5) (width 0.25) (layer "F.Cu") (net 16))
 (segment (start 65.01 93.5) (end 65 93.49) (width 0.25) (layer "F.Cu") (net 16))
 (segment (start 63.71 93.49) (end 62.8 94.4) (width 0.25) (layer "F.Cu") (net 16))
 (segment (start 65 93.49) (end 63.71 93.49) (width 0.25) (layer "F.Cu") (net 16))
 (segment (start 62.8 94.4) (end 62.8 95.8625) (width 0.25) (layer "F.Cu") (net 16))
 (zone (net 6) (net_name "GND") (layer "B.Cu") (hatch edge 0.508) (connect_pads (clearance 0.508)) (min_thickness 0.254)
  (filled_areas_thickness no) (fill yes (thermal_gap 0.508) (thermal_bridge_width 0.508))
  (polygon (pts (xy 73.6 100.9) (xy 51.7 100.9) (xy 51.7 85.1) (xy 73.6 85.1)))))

